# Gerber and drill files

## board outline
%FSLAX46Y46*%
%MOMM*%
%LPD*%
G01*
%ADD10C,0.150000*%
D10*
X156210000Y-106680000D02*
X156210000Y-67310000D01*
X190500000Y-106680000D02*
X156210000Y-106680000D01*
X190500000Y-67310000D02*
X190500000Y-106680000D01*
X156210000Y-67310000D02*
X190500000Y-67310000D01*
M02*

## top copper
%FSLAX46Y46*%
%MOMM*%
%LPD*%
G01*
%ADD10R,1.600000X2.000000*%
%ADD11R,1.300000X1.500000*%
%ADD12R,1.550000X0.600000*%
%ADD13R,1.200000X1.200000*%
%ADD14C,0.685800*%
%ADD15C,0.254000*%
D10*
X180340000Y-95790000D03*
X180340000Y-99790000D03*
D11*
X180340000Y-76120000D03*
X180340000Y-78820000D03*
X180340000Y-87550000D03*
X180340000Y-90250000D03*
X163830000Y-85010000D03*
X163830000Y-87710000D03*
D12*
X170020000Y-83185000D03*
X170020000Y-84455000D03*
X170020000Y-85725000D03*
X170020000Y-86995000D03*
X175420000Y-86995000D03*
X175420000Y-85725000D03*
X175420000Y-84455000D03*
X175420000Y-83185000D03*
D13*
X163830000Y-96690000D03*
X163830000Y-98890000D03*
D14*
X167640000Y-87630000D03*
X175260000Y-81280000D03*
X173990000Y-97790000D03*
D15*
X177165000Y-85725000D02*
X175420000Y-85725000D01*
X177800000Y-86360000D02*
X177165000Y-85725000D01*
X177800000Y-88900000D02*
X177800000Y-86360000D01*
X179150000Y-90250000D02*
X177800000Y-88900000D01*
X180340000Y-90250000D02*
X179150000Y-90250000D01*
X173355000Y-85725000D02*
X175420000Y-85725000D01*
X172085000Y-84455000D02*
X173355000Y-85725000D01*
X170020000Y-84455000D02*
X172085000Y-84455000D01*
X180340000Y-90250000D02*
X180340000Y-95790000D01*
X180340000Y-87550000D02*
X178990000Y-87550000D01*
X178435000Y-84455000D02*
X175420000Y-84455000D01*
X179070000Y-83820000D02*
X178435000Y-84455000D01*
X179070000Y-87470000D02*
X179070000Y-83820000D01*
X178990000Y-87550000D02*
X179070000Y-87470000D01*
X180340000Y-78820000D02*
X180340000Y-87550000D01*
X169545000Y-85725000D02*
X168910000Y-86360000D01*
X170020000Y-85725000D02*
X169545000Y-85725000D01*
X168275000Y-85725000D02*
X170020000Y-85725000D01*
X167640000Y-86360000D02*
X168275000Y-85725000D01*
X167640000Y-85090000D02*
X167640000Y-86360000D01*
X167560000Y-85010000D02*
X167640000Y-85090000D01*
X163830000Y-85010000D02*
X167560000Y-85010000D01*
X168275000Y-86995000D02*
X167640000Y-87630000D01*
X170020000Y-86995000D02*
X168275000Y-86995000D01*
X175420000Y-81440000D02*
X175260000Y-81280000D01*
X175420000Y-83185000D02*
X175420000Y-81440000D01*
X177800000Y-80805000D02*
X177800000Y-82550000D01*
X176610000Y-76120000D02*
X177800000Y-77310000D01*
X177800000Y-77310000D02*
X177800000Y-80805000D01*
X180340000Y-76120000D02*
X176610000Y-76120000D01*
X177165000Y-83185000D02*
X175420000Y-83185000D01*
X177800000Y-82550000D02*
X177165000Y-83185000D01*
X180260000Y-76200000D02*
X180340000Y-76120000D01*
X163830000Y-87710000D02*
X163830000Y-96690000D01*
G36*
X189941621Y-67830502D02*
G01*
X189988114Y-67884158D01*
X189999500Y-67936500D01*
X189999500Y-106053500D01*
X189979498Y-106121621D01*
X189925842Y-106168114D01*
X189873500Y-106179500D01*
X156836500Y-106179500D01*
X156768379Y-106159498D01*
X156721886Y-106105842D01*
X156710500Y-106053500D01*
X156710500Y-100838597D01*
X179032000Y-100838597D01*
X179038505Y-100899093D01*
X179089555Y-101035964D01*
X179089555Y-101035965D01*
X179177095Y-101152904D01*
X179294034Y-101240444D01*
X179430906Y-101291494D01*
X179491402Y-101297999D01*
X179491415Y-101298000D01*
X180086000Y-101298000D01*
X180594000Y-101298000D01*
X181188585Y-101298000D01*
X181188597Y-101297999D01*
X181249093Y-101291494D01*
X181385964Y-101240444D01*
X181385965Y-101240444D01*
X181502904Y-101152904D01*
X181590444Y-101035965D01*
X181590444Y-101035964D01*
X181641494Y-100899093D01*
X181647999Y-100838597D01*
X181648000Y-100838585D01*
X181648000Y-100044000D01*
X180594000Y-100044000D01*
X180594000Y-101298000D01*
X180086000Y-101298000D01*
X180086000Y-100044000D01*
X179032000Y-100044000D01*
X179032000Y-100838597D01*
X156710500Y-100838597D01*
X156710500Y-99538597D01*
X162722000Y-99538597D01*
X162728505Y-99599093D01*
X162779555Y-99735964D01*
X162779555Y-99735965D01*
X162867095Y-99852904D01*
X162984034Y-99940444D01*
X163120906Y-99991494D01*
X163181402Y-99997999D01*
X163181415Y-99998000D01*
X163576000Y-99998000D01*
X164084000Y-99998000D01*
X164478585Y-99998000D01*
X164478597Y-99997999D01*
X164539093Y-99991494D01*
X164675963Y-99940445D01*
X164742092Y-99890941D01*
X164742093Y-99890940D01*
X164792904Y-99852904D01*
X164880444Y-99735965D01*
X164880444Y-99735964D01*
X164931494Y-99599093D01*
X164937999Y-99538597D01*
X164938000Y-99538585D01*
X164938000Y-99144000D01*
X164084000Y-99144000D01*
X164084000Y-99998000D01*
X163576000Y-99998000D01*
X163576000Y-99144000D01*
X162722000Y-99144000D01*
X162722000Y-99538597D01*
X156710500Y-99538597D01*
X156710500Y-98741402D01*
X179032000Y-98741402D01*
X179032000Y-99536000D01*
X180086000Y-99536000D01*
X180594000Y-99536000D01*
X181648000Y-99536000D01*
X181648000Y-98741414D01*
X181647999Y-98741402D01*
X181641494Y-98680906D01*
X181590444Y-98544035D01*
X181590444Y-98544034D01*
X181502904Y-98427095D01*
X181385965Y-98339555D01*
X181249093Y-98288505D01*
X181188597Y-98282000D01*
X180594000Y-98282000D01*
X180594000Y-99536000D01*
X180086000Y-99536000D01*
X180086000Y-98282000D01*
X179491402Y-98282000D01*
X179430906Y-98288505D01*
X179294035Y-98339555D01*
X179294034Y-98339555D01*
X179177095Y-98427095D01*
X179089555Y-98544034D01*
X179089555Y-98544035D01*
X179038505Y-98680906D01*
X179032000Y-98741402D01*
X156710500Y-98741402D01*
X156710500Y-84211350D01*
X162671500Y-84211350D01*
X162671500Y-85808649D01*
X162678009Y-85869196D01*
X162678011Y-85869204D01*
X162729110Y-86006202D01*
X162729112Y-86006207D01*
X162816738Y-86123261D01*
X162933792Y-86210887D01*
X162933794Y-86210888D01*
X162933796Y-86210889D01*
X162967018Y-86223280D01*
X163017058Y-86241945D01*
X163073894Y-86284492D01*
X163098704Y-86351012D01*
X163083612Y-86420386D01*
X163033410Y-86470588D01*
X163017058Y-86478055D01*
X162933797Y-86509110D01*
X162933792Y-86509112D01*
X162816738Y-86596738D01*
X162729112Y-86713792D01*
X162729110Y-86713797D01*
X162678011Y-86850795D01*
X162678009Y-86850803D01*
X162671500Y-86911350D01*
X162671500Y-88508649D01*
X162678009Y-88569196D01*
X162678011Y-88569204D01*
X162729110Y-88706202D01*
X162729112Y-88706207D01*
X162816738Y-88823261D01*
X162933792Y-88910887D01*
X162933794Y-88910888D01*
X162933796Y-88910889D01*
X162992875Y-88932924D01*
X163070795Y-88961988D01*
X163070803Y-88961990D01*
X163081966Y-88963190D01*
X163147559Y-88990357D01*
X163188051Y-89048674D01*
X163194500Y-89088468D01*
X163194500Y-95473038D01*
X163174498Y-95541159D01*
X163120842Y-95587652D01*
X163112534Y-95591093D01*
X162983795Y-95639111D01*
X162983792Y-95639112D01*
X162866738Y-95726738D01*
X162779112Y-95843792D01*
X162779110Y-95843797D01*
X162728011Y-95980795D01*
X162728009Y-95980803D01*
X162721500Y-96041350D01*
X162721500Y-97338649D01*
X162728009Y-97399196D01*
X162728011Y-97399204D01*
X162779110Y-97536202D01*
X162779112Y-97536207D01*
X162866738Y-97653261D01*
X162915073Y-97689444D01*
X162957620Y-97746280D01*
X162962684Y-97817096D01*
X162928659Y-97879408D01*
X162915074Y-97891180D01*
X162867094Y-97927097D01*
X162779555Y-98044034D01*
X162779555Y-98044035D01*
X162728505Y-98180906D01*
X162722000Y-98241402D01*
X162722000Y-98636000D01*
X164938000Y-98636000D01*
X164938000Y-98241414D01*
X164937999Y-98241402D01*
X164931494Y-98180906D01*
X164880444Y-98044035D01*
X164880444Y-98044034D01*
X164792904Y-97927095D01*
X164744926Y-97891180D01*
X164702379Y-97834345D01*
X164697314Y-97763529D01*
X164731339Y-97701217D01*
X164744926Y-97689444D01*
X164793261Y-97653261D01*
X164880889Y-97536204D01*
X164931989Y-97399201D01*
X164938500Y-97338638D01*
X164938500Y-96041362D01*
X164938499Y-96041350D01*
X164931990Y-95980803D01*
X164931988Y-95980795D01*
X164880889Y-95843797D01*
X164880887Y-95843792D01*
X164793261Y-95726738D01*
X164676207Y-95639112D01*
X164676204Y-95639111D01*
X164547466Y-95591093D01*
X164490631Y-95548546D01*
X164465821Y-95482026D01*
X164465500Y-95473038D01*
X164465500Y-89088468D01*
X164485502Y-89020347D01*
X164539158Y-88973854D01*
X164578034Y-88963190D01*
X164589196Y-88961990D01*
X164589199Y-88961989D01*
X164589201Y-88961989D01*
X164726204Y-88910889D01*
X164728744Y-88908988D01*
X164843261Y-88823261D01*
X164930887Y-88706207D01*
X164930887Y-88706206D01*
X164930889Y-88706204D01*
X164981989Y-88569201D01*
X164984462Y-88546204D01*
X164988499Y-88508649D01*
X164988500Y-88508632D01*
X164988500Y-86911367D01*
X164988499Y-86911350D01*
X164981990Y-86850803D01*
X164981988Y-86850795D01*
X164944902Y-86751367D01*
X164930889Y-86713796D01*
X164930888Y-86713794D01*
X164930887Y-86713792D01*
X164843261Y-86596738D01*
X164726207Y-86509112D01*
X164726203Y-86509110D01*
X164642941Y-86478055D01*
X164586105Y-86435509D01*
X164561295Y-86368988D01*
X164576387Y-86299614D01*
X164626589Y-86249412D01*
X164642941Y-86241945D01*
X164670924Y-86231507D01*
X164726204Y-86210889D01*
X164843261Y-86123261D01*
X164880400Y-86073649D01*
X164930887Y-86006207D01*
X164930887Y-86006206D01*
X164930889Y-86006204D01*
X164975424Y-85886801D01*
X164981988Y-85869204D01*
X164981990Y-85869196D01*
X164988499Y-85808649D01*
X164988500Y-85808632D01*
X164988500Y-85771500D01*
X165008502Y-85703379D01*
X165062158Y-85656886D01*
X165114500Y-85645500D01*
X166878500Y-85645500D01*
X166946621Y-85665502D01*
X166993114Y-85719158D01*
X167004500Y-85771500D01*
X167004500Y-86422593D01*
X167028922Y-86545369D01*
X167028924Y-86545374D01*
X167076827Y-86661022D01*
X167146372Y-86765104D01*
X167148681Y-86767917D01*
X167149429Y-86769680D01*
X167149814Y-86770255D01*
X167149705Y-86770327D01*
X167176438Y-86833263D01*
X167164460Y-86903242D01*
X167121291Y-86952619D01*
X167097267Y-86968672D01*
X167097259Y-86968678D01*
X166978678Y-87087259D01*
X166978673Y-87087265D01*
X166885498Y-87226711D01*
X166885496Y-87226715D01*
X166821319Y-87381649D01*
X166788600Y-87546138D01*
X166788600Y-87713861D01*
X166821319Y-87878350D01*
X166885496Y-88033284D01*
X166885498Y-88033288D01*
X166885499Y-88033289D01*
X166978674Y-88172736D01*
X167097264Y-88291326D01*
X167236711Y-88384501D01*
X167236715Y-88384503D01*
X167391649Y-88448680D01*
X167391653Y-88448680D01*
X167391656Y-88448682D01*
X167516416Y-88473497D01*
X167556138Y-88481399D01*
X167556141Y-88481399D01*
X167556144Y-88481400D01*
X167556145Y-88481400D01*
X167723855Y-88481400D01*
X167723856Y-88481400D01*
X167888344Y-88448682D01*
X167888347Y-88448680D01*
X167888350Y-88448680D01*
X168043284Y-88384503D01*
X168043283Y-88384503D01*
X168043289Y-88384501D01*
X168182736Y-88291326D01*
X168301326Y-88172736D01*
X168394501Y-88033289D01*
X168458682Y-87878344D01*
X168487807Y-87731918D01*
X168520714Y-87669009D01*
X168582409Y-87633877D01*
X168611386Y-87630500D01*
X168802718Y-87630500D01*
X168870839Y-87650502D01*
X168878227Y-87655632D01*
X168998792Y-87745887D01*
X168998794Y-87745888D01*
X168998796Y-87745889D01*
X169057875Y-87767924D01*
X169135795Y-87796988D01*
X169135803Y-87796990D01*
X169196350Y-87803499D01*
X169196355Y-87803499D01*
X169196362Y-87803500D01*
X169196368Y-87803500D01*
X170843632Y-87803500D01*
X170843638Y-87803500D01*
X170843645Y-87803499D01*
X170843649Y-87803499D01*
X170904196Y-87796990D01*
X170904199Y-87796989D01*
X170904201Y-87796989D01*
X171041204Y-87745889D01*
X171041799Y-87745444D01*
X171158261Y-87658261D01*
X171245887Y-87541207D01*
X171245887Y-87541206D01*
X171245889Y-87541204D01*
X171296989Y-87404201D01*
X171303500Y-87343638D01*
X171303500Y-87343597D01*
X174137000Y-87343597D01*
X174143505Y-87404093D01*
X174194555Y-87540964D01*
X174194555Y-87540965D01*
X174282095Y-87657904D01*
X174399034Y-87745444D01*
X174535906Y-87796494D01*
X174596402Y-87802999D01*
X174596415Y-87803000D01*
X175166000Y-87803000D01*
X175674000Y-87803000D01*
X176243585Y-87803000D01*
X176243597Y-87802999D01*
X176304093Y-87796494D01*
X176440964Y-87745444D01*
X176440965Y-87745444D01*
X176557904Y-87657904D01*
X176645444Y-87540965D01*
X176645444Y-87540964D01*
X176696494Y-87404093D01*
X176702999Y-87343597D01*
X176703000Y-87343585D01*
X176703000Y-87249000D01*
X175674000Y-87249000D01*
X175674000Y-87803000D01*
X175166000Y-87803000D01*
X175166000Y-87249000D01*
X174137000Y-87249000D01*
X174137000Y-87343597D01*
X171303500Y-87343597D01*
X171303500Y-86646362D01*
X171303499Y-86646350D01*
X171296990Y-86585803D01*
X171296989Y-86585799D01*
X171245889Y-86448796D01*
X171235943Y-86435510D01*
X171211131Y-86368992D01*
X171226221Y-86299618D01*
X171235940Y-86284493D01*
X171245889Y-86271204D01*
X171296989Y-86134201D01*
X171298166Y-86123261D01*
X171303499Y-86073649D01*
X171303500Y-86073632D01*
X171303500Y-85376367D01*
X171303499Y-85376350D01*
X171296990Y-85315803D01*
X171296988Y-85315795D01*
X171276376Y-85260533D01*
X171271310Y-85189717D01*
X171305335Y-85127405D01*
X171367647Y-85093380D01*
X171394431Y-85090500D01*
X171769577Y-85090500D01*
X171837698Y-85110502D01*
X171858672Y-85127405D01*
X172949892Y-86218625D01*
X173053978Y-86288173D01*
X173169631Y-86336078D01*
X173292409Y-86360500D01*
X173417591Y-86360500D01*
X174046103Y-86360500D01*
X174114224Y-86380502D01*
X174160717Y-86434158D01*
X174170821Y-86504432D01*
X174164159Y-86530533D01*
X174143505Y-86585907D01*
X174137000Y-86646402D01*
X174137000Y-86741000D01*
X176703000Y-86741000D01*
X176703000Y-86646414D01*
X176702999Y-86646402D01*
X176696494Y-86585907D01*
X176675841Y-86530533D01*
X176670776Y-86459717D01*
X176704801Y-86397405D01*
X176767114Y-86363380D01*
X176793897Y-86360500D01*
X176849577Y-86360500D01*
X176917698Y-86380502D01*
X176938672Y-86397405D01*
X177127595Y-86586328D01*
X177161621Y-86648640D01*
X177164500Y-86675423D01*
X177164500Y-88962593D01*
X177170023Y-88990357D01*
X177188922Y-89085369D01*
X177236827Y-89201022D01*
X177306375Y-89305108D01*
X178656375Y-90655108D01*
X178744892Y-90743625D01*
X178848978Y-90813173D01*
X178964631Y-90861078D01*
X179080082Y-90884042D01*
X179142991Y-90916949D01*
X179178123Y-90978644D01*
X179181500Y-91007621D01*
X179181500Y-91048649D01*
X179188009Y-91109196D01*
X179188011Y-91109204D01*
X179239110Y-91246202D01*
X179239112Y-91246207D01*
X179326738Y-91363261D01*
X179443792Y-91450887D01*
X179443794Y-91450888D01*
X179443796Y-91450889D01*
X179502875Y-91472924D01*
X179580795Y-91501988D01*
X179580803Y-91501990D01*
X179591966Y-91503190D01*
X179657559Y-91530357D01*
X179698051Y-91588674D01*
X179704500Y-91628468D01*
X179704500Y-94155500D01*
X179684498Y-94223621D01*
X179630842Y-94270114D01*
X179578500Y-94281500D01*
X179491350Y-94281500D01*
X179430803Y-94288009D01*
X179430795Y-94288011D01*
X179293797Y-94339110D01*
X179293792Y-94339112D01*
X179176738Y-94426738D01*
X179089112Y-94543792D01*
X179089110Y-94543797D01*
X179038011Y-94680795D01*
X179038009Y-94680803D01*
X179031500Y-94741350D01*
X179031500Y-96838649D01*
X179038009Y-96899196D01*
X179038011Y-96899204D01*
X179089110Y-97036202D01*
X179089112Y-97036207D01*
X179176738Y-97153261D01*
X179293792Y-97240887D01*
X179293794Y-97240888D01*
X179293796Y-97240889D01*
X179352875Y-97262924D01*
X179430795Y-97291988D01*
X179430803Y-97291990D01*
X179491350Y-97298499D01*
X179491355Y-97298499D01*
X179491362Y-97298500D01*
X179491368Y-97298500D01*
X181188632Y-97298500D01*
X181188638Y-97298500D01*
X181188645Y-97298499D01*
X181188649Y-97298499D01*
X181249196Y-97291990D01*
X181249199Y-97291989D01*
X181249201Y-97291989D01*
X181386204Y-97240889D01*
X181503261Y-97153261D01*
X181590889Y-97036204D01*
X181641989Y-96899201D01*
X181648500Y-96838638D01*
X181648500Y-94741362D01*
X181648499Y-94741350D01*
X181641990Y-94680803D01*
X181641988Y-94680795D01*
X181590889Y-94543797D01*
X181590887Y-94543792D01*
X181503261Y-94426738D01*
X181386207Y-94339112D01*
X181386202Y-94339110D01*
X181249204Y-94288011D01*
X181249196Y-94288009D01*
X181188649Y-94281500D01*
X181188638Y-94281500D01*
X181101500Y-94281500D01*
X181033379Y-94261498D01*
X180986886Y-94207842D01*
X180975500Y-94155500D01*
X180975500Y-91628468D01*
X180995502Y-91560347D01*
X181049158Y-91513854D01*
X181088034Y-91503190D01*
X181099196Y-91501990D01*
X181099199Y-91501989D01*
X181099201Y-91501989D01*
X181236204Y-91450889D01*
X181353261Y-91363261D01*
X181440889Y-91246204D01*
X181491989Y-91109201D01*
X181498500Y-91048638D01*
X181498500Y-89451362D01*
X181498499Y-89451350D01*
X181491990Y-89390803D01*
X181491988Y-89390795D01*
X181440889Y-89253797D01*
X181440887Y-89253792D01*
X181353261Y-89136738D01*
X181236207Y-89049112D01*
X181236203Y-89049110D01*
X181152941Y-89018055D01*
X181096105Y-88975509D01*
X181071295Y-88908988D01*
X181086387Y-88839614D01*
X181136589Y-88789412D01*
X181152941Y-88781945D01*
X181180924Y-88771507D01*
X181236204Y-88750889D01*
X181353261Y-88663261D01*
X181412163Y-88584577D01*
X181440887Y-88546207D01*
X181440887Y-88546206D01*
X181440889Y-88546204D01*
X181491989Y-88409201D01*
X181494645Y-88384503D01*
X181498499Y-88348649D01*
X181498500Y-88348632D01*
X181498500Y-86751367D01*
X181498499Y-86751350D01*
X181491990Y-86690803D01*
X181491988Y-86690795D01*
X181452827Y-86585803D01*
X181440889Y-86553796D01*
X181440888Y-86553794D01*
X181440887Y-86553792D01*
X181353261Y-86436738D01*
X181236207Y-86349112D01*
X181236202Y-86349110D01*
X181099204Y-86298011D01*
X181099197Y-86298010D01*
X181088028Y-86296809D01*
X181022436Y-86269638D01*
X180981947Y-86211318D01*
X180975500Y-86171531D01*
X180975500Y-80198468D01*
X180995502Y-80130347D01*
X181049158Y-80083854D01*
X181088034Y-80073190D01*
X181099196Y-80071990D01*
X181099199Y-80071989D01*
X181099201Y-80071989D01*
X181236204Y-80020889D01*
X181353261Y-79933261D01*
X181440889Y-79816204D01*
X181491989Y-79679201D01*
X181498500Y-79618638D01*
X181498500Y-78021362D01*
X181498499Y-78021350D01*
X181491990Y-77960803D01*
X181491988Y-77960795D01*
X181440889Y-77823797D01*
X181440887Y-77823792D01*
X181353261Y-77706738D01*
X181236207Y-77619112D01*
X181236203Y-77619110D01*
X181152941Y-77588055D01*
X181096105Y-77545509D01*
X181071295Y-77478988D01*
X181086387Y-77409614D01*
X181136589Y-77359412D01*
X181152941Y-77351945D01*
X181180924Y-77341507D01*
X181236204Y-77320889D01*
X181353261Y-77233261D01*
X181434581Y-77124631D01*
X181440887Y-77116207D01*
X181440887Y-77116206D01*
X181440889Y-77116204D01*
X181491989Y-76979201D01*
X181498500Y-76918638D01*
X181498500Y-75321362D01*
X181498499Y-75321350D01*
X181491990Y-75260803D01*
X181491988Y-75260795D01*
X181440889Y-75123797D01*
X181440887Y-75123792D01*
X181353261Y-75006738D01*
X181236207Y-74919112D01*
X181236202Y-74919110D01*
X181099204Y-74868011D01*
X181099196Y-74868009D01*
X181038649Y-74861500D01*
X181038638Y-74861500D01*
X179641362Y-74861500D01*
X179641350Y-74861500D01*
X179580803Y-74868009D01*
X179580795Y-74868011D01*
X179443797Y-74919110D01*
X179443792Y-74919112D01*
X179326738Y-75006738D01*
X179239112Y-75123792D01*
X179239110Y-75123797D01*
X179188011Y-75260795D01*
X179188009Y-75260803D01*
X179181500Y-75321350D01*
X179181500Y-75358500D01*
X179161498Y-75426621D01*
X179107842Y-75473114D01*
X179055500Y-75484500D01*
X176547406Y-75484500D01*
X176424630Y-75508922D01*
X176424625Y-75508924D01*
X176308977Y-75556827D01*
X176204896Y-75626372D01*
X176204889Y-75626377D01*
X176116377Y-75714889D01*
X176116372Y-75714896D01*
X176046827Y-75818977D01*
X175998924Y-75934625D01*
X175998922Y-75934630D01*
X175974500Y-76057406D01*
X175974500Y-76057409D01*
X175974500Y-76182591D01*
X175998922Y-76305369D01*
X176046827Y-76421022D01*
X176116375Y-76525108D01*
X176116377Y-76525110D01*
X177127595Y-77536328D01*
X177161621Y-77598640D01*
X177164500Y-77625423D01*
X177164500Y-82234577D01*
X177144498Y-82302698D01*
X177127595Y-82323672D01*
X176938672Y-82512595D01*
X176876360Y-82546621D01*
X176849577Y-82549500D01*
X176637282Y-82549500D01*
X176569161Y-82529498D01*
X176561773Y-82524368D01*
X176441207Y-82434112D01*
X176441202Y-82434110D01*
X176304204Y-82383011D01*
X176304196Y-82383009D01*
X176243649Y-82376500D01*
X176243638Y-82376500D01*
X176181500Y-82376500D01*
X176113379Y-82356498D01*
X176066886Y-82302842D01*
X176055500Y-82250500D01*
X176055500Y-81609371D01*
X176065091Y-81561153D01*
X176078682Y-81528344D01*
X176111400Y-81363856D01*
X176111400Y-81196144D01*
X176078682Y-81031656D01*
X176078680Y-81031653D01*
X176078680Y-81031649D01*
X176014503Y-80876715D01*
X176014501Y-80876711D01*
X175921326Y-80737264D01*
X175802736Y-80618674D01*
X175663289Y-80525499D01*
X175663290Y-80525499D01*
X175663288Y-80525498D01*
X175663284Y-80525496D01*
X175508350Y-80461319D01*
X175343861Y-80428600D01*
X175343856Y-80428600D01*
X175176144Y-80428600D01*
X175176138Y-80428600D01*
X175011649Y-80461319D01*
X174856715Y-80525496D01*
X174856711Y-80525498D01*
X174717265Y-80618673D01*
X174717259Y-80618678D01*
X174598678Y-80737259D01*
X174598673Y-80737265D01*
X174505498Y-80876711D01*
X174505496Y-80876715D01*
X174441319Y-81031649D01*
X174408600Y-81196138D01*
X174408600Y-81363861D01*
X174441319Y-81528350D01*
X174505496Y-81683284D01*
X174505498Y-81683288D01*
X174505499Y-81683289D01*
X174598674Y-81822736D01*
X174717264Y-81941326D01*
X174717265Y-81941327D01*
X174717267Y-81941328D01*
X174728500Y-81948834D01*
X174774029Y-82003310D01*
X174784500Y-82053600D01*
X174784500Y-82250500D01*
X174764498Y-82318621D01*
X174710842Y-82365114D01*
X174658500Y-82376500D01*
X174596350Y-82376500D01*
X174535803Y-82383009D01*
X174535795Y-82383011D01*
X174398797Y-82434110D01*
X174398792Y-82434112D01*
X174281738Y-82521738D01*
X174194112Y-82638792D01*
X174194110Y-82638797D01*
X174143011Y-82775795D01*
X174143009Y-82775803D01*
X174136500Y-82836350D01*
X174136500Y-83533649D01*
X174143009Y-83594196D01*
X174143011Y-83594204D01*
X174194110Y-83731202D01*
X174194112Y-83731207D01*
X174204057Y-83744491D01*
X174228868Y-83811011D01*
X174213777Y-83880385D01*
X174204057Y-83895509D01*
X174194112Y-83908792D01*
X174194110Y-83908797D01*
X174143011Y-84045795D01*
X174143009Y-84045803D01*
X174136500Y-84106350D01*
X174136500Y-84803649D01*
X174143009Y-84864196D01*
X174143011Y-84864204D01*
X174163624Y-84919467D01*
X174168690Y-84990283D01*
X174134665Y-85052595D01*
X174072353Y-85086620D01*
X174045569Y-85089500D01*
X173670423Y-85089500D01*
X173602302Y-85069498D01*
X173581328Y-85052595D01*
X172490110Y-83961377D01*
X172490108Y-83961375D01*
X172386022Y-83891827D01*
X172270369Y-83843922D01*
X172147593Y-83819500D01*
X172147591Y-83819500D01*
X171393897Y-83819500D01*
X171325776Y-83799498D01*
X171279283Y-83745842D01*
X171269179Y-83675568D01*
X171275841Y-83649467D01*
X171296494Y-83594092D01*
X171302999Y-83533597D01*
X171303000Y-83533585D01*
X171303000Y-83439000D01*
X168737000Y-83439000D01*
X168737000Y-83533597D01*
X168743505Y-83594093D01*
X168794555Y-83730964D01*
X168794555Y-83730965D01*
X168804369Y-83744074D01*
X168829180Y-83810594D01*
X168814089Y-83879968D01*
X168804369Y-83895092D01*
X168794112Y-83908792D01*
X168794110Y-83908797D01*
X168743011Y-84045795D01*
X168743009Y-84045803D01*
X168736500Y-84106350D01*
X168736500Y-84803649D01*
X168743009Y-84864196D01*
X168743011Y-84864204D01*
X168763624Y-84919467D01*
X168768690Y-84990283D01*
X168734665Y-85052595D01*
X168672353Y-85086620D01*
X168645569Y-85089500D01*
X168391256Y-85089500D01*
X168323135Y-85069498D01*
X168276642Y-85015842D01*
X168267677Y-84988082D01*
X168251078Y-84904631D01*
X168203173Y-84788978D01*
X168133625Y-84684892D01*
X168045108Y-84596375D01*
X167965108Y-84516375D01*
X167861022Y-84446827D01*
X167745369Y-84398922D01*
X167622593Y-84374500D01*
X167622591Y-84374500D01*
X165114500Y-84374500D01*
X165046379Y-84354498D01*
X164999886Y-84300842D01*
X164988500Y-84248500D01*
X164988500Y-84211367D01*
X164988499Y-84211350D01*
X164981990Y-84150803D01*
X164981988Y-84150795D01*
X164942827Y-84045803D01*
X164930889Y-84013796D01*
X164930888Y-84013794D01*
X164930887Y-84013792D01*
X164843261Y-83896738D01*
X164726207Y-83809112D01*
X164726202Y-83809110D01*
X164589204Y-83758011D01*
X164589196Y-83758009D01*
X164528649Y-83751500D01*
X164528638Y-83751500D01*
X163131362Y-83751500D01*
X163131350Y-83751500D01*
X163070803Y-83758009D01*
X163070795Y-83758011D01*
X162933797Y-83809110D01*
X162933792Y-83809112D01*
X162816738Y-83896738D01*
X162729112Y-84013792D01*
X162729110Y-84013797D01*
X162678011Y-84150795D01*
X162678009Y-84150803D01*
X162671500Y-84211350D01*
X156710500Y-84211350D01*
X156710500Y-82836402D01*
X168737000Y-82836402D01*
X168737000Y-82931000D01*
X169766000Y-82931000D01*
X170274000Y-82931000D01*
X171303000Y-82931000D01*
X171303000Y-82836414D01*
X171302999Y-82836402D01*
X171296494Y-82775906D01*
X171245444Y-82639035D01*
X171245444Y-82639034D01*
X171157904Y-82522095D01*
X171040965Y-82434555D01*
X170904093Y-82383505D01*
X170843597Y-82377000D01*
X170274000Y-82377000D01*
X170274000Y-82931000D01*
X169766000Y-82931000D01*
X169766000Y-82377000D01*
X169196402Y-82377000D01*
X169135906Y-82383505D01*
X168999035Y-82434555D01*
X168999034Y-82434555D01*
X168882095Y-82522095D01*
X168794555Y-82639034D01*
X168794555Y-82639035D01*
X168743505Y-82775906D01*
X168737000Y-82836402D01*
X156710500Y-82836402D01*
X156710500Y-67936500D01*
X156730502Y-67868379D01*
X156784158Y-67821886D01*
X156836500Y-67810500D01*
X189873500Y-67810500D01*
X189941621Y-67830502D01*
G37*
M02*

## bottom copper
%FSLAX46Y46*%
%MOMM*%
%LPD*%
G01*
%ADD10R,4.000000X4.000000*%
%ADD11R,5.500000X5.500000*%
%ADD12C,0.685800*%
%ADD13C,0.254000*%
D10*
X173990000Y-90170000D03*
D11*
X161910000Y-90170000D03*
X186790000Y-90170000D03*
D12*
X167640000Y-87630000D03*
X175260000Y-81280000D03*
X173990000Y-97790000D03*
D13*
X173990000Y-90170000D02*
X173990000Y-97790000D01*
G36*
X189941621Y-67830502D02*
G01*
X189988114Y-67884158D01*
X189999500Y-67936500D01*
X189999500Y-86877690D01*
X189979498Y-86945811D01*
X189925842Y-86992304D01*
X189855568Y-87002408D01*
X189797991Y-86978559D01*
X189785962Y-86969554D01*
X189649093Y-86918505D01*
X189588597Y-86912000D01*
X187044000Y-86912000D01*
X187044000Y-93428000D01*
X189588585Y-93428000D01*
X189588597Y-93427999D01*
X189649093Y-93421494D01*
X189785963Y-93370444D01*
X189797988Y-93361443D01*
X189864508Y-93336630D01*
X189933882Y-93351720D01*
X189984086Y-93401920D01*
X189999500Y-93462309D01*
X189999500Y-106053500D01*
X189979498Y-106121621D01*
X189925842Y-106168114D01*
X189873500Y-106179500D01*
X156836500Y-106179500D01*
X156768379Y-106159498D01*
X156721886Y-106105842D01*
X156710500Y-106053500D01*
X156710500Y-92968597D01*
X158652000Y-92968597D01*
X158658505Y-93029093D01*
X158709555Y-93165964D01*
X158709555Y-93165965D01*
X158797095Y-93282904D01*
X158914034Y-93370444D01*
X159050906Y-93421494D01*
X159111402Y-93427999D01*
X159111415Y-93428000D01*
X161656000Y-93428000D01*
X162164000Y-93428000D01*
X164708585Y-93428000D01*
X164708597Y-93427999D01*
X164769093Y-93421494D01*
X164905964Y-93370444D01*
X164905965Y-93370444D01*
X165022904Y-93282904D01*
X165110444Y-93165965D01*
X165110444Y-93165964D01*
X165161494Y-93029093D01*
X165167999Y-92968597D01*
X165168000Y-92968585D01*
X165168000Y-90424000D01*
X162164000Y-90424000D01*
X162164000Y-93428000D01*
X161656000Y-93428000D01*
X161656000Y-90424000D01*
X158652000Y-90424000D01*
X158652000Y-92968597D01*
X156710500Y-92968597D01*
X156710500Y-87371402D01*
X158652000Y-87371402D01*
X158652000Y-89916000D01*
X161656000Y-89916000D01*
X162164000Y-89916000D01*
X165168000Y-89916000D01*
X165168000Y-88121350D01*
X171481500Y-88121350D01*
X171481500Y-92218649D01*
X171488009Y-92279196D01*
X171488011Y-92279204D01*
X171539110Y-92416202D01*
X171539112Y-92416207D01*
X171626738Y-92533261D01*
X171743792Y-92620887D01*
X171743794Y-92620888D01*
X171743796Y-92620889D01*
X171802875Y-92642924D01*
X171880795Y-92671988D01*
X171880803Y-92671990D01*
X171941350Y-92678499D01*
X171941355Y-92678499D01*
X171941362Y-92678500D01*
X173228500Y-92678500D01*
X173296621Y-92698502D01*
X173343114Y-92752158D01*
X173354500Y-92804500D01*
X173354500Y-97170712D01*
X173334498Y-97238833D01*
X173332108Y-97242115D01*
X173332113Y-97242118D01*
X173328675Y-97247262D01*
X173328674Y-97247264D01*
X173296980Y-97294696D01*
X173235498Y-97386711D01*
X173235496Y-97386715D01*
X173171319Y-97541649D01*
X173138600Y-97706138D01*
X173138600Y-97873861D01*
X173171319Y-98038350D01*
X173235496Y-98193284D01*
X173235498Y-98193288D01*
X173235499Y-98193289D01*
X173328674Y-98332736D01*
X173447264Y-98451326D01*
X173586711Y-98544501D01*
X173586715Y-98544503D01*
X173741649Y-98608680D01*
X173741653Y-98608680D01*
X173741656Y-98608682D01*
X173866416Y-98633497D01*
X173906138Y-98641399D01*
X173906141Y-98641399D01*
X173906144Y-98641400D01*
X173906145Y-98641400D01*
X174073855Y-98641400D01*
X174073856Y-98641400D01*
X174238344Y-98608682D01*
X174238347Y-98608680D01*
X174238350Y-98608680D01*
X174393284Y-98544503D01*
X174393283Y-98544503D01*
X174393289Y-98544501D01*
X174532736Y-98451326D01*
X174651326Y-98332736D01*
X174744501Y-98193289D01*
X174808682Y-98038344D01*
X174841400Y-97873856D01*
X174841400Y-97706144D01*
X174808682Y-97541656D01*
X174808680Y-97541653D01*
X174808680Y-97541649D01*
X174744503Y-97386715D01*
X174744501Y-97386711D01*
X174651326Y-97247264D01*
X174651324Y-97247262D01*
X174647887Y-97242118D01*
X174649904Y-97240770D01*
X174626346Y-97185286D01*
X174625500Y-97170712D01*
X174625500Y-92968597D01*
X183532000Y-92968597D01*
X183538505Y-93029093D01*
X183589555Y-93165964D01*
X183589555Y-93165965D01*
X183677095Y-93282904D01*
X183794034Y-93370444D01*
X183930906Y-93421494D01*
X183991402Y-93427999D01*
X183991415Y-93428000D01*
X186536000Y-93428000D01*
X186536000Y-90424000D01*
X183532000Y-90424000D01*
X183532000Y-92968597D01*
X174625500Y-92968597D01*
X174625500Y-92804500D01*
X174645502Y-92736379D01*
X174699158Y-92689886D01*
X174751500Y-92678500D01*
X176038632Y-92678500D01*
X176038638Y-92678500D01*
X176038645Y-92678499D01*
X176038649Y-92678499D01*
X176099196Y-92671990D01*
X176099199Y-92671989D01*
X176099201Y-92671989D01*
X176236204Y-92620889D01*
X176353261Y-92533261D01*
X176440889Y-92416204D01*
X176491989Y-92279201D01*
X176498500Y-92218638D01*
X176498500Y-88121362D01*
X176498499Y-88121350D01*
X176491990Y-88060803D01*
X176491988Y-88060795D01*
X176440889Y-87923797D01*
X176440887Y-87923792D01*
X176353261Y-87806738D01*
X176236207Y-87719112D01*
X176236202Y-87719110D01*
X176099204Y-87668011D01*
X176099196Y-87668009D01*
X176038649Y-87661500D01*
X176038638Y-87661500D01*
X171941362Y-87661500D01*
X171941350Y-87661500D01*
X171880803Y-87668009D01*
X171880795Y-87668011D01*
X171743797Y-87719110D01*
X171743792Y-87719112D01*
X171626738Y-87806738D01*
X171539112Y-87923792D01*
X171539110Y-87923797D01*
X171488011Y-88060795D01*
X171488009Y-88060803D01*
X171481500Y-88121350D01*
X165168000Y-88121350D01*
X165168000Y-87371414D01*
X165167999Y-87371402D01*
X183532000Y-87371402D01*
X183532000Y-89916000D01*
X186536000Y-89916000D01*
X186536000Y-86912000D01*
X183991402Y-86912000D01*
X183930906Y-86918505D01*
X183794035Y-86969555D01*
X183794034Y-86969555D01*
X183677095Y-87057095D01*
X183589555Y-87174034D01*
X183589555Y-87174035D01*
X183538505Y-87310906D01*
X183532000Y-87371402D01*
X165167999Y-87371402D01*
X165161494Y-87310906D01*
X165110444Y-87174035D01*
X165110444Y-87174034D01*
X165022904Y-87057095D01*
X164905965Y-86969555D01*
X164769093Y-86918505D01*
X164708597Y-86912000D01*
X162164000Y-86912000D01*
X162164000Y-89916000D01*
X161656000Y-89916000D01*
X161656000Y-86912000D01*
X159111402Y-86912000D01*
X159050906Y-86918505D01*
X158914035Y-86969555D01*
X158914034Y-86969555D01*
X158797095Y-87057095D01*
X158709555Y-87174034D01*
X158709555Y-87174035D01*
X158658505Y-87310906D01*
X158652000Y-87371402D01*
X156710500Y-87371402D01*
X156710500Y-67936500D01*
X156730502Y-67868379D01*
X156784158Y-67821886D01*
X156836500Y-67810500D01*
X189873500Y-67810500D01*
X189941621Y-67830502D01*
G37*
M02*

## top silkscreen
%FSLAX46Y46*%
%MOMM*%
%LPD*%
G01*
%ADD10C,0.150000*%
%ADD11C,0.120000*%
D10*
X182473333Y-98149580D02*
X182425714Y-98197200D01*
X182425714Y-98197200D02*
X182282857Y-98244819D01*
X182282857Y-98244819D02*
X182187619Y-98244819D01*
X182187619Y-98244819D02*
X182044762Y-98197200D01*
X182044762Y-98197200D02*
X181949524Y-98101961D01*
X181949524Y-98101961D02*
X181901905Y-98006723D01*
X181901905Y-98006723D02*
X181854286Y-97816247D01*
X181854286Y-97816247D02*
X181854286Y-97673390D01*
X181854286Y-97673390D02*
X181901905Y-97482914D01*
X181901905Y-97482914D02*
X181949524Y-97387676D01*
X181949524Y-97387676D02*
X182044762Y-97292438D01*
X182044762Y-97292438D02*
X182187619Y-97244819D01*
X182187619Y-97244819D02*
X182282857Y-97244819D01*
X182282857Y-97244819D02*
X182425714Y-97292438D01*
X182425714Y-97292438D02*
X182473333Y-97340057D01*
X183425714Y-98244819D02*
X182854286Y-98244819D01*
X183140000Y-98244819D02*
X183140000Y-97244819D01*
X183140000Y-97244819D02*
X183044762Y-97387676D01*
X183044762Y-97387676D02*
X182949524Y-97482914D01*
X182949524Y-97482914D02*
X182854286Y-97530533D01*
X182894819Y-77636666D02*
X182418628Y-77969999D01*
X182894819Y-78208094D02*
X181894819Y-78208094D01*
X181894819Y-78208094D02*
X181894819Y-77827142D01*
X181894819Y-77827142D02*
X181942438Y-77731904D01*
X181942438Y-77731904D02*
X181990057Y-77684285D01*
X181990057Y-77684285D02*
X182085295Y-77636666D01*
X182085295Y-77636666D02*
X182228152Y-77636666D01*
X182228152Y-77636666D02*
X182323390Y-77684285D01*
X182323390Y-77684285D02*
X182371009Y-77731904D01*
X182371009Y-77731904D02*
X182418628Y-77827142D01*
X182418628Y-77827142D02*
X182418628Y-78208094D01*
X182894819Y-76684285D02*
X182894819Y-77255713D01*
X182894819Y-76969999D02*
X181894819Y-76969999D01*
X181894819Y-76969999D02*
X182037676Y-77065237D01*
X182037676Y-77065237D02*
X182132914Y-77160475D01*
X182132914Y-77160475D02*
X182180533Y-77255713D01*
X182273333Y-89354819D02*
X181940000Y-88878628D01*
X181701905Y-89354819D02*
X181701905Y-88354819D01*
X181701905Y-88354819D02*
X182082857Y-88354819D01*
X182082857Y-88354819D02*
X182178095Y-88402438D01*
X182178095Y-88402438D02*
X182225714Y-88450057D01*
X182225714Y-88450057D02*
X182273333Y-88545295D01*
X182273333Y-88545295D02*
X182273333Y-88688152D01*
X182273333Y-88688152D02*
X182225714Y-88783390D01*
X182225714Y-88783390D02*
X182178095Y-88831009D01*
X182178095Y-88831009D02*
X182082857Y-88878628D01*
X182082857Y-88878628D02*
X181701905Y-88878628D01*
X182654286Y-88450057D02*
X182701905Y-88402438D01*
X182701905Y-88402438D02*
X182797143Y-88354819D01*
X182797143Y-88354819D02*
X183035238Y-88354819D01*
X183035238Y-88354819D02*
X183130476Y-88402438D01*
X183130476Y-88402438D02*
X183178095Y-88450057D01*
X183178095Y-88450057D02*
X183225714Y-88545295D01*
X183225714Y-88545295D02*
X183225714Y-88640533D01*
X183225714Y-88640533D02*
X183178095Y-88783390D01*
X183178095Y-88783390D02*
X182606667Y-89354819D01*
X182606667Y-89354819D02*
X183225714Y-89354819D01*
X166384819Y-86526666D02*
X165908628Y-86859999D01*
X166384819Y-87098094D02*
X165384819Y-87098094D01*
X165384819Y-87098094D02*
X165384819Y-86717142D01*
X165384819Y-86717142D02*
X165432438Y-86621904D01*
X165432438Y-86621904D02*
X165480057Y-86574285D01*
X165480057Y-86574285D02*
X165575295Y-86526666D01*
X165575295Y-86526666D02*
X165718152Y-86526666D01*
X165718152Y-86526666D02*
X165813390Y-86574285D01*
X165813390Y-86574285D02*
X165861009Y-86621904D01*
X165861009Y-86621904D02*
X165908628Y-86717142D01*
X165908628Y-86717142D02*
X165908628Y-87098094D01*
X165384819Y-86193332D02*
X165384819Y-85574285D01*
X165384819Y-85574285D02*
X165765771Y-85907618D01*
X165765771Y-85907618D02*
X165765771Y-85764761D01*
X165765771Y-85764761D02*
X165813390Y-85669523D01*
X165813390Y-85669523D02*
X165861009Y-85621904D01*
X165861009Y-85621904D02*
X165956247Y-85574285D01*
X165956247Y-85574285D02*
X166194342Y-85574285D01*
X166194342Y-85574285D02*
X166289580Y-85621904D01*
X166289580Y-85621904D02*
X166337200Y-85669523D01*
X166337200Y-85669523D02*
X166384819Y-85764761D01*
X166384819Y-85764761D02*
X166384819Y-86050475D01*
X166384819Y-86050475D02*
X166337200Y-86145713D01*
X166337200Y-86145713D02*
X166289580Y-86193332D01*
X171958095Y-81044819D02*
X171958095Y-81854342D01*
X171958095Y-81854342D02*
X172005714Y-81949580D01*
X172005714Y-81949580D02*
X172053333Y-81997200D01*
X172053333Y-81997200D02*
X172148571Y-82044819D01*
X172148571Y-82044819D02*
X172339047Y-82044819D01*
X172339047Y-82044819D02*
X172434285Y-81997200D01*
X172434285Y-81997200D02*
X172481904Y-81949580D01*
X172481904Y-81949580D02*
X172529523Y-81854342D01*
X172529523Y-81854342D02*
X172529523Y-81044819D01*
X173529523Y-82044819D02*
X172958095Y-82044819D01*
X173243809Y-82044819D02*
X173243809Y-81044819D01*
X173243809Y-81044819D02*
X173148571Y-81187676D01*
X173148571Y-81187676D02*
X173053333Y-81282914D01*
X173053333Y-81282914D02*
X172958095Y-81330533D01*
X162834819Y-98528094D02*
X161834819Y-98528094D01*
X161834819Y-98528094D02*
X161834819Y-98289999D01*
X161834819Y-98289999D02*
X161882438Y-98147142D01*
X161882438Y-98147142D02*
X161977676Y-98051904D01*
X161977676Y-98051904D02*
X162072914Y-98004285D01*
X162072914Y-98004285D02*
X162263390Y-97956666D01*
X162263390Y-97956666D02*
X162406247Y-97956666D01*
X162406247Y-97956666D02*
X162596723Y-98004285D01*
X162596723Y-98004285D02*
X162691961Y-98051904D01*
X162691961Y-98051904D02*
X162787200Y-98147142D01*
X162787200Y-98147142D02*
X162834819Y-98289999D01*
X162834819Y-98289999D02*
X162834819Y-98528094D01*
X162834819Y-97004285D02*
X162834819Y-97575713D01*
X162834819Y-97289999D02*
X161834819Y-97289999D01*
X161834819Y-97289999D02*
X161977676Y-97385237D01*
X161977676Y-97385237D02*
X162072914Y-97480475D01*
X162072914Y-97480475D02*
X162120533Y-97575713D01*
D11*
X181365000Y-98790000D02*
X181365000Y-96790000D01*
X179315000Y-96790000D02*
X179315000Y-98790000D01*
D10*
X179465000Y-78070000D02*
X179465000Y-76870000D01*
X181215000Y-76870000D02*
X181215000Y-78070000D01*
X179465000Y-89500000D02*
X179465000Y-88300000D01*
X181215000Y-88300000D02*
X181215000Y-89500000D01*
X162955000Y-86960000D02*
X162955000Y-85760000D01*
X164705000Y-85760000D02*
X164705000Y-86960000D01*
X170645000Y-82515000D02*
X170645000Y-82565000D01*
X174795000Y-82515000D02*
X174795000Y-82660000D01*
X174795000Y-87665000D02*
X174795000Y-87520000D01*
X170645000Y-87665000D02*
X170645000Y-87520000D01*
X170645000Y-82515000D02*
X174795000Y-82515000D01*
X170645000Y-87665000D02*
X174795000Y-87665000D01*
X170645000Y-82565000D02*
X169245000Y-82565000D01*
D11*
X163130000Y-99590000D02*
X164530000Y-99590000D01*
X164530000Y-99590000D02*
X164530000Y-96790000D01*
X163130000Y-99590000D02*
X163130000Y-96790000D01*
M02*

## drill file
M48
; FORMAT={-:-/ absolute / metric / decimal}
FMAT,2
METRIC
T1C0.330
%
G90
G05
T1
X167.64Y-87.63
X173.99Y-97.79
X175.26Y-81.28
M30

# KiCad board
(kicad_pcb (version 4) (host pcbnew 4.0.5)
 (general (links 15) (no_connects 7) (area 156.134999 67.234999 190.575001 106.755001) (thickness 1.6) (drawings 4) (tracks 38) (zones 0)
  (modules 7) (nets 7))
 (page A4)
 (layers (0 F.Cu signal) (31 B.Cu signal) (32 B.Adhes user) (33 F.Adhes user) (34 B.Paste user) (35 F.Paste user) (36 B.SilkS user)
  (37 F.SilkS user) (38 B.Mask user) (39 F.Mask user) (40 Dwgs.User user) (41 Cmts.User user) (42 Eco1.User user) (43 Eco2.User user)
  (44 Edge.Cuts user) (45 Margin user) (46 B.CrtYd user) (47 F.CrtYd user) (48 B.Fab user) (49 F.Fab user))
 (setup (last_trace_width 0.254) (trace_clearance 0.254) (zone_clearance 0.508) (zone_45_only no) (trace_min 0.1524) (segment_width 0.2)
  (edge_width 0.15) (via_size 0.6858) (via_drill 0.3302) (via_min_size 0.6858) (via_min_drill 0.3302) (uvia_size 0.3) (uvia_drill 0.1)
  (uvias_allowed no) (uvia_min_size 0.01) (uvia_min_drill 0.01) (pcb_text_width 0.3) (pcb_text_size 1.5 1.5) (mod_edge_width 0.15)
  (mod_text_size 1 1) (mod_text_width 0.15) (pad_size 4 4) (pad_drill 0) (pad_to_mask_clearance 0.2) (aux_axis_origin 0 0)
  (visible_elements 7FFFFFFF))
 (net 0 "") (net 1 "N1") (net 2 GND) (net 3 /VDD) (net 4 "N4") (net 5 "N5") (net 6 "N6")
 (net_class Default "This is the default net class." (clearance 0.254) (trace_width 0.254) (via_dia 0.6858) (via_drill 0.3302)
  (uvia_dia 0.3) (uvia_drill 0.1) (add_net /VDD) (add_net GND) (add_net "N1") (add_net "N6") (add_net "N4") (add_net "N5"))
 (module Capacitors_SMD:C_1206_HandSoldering (layer F.Cu) (at 180.34 97.79 270)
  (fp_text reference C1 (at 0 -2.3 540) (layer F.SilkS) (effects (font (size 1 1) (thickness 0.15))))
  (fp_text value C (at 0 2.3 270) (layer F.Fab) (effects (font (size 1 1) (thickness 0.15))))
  (fp_line (start 1 -1.025) (end -1 -1.025) (layer F.SilkS) (width 0.12))
  (fp_line (start -1 1.025) (end 1 1.025) (layer F.SilkS) (width 0.12))
  (pad 1 smd rect (at -2 0 270) (size 2 1.6) (layers F.Cu F.Paste F.Mask) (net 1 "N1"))
  (pad 2 smd rect (at 2 0 270) (size 2 1.6) (layers F.Cu F.Paste F.Mask) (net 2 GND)))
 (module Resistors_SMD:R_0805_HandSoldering (layer F.Cu) (at 180.34 77.47 270)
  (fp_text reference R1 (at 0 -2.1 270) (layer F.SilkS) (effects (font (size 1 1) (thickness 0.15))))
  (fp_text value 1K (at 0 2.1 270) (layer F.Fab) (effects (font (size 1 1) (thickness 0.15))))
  (fp_line (start 0.6 0.875) (end -0.6 0.875) (layer F.SilkS) (width 0.15))
  (fp_line (start -0.6 -0.875) (end 0.6 -0.875) (layer F.SilkS) (width 0.15))
  (pad 1 smd rect (at -1.35 0 270) (size 1.5 1.3) (layers F.Cu F.Paste F.Mask) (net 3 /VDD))
  (pad 2 smd rect (at 1.35 0 270) (size 1.5 1.3) (layers F.Cu F.Paste F.Mask) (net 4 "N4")))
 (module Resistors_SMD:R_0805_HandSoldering (layer F.Cu) (at 180.34 88.9 270)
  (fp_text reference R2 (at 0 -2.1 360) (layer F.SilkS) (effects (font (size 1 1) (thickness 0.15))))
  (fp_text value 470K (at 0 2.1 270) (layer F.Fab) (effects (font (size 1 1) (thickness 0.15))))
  (fp_line (start 0.6 0.875) (end -0.6 0.875) (layer F.SilkS) (width 0.15))
  (fp_line (start -0.6 -0.875) (end 0.6 -0.875) (layer F.SilkS) (width 0.15))
  (pad 1 smd rect (at -1.35 0 270) (size 1.5 1.3) (layers F.Cu F.Paste F.Mask) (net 4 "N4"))
  (pad 2 smd rect (at 1.35 0 270) (size 1.5 1.3) (layers F.Cu F.Paste F.Mask) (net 1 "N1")))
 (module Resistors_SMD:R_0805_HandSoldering (layer F.Cu) (at 163.83 86.36 270)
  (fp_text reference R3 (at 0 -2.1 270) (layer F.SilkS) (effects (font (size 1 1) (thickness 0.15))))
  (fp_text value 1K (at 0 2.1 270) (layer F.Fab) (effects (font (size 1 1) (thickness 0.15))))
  (fp_line (start 0.6 0.875) (end -0.6 0.875) (layer F.SilkS) (width 0.15))
  (fp_line (start -0.6 -0.875) (end 0.6 -0.875) (layer F.SilkS) (width 0.15))
  (pad 1 smd rect (at -1.35 0 270) (size 1.5 1.3) (layers F.Cu F.Paste F.Mask) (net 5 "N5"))
  (pad 2 smd rect (at 1.35 0 270) (size 1.5 1.3) (layers F.Cu F.Paste F.Mask) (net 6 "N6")))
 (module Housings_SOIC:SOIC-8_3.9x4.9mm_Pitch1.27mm (layer F.Cu) (at 172.72 85.09)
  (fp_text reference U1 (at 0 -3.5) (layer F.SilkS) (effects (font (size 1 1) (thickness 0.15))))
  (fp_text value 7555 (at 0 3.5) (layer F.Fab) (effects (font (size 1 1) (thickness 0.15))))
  (fp_line (start -2.075 -2.575) (end -2.075 -2.525) (layer F.SilkS) (width 0.15))
  (fp_line (start 2.075 -2.575) (end 2.075 -2.43) (layer F.SilkS) (width 0.15))
  (fp_line (start 2.075 2.575) (end 2.075 2.43) (layer F.SilkS) (width 0.15))
  (fp_line (start -2.075 2.575) (end -2.075 2.43) (layer F.SilkS) (width 0.15))
  (fp_line (start -2.075 -2.575) (end 2.075 -2.575) (layer F.SilkS) (width 0.15))
  (fp_line (start -2.075 2.575) (end 2.075 2.575) (layer F.SilkS) (width 0.15))
  (fp_line (start -2.075 -2.525) (end -3.475 -2.525) (layer F.SilkS) (width 0.15))
  (pad 1 smd rect (at -2.7 -1.905) (size 1.55 0.6) (layers F.Cu F.Paste F.Mask) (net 2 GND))
  (pad 2 smd rect (at -2.7 -0.635) (size 1.55 0.6) (layers F.Cu F.Paste F.Mask) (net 1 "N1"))
  (pad 3 smd rect (at -2.7 0.635) (size 1.55 0.6) (layers F.Cu F.Paste F.Mask) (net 5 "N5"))
  (pad 4 smd rect (at -2.7 1.905) (size 1.55 0.6) (layers F.Cu F.Paste F.Mask) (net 3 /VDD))
  (pad 5 smd rect (at 2.7 1.905) (size 1.55 0.6) (layers F.Cu F.Paste F.Mask) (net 2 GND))
  (pad 6 smd rect (at 2.7 0.635) (size 1.55 0.6) (layers F.Cu F.Paste F.Mask) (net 1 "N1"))
  (pad 7 smd rect (at 2.7 -0.635) (size 1.55 0.6) (layers F.Cu F.Paste F.Mask) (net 4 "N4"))
  (pad 8 smd rect (at 2.7 -1.905) (size 1.55 0.6) (layers F.Cu F.Paste F.Mask) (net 3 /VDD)))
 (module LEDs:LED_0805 (layer F.Cu) (at 163.83 97.79 90)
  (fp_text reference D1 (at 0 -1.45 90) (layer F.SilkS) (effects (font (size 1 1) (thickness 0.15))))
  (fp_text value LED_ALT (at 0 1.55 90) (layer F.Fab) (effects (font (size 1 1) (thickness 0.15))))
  (fp_line (start -1.8 -0.7) (end -1.8 0.7) (layer F.SilkS) (width 0.12))
  (fp_line (start -1.8 0.7) (end 1 0.7) (layer F.SilkS) (width 0.12))
  (fp_line (start -1.8 -0.7) (end 1 -0.7) (layer F.SilkS) (width 0.12))
  (pad 2 smd rect (at 1.1 0 270) (size 1.2 1.2) (layers F.Cu F.Paste F.Mask) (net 6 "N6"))
  (pad 1 smd rect (at -1.1 0 270) (size 1.2 1.2) (layers F.Cu F.Paste F.Mask) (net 2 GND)))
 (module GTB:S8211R (layer B.Cu) (at 173.99 90.17)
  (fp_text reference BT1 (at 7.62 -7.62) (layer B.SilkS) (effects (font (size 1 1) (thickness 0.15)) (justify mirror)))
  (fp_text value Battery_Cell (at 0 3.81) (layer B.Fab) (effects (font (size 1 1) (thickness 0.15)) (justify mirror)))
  (pad 2 smd rect (at 0 0) (size 4 4) (layers B.Cu B.Paste B.Mask) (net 2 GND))
  (pad 1 smd rect (at -12.08 0) (size 5.5 5.5) (layers B.Cu B.Paste B.Mask) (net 3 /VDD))
  (pad 1 smd rect (at 12.8 0) (size 5.5 5.5) (layers B.Cu B.Paste B.Mask) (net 3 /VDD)))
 (gr_line (start 156.21 106.68) (end 156.21 67.31) (angle 90) (layer Edge.Cuts) (width 0.15))
 (gr_line (start 190.5 106.68) (end 156.21 106.68) (angle 90) (layer Edge.Cuts) (width 0.15))
 (gr_line (start 190.5 67.31) (end 190.5 106.68) (angle 90) (layer Edge.Cuts) (width 0.15))
 (gr_line (start 156.21 67.31) (end 190.5 67.31) (angle 90) (layer Edge.Cuts) (width 0.15))
 (segment (start 177.165 85.725) (end 175.42 85.725) (width 0.254) (layer F.Cu) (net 1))
 (segment (start 177.8 86.36) (end 177.165 85.725) (width 0.254) (layer F.Cu) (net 1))
 (segment (start 177.8 88.9) (end 177.8 86.36) (width 0.254) (layer F.Cu) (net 1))
 (segment (start 179.15 90.25) (end 177.8 88.9) (width 0.254) (layer F.Cu) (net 1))
 (segment (start 180.34 90.25) (end 179.15 90.25) (width 0.254) (layer F.Cu) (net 1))
 (segment (start 173.355 85.725) (end 175.42 85.725) (width 0.254) (layer F.Cu) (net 1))
 (segment (start 172.085 84.455) (end 173.355 85.725) (width 0.254) (layer F.Cu) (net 1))
 (segment (start 170.02 84.455) (end 172.085 84.455) (width 0.254) (layer F.Cu) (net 1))
 (segment (start 180.34 90.25) (end 180.34 95.79) (width 0.254) (layer F.Cu) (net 1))
 (segment (start 180.34 87.55) (end 178.99 87.55) (width 0.254) (layer F.Cu) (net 4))
 (segment (start 178.435 84.455) (end 175.42 84.455) (width 0.254) (layer F.Cu) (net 4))
 (segment (start 179.07 83.82) (end 178.435 84.455) (width 0.254) (layer F.Cu) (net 4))
 (segment (start 179.07 87.47) (end 179.07 83.82) (width 0.254) (layer F.Cu) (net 4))
 (segment (start 178.99 87.55) (end 179.07 87.47) (width 0.254) (layer F.Cu) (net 4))
 (segment (start 180.34 78.82) (end 180.34 87.55) (width 0.254) (layer F.Cu) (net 4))
 (segment (start 169.545 85.725) (end 168.91 86.36) (width 0.254) (layer F.Cu) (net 5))
 (segment (start 170.02 85.725) (end 169.545 85.725) (width 0.254) (layer F.Cu) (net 5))
 (segment (start 168.275 85.725) (end 170.02 85.725) (width 0.254) (layer F.Cu) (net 5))
 (segment (start 167.64 86.36) (end 168.275 85.725) (width 0.254) (layer F.Cu) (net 5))
 (segment (start 167.64 85.09) (end 167.64 86.36) (width 0.254) (layer F.Cu) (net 5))
 (segment (start 167.56 85.01) (end 167.64 85.09) (width 0.254) (layer F.Cu) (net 5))
 (segment (start 163.83 85.01) (end 167.56 85.01) (width 0.254) (layer F.Cu) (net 5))
 (via (at 167.64 87.63) (size 0.6858) (drill 0.3302) (layers F.Cu B.Cu) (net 3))
 (segment (start 168.275 86.995) (end 167.64 87.63) (width 0.254) (layer F.Cu) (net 3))
 (segment (start 170.02 86.995) (end 168.275 86.995) (width 0.254) (layer F.Cu) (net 3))
 (via (at 175.26 81.28) (size 0.6858) (drill 0.3302) (layers F.Cu B.Cu) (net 3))
 (segment (start 175.42 81.44) (end 175.26 81.28) (width 0.254) (layer F.Cu) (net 3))
 (segment (start 175.42 83.185) (end 175.42 81.44) (width 0.254) (layer F.Cu) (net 3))
 (segment (start 177.8 80.805) (end 177.8 82.55) (width 0.254) (layer F.Cu) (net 3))
 (segment (start 176.61 76.12) (end 177.8 77.31) (width 0.254) (layer F.Cu) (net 3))
 (segment (start 177.8 77.31) (end 177.8 80.805) (width 0.254) (layer F.Cu) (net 3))
 (segment (start 180.34 76.12) (end 176.61 76.12) (width 0.254) (layer F.Cu) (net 3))
 (segment (start 177.165 83.185) (end 175.42 83.185) (width 0.254) (layer F.Cu) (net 3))
 (segment (start 177.8 82.55) (end 177.165 83.185) (width 0.254) (layer F.Cu) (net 3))
 (segment (start 180.26 76.2) (end 180.34 76.12) (width 0.254) (layer F.Cu) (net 3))
 (segment (start 173.99 90.17) (end 173.99 97.79) (width 0.254) (layer B.Cu) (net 2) (status 400010))
 (via (at 173.99 97.79) (size 0.6858) (drill 0.3302) (layers F.Cu B.Cu) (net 2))
 (segment (start 163.83 87.71) (end 163.83 96.69) (width 0.254) (layer F.Cu) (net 6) (status 10))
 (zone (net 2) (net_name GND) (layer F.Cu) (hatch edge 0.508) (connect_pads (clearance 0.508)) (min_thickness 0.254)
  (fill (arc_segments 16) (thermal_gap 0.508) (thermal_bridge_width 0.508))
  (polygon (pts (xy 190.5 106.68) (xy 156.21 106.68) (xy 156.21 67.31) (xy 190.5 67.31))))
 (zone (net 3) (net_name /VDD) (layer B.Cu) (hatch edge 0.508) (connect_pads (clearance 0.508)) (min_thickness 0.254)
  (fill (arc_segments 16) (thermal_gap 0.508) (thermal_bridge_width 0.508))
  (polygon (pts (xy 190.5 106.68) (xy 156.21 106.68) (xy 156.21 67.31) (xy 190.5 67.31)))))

